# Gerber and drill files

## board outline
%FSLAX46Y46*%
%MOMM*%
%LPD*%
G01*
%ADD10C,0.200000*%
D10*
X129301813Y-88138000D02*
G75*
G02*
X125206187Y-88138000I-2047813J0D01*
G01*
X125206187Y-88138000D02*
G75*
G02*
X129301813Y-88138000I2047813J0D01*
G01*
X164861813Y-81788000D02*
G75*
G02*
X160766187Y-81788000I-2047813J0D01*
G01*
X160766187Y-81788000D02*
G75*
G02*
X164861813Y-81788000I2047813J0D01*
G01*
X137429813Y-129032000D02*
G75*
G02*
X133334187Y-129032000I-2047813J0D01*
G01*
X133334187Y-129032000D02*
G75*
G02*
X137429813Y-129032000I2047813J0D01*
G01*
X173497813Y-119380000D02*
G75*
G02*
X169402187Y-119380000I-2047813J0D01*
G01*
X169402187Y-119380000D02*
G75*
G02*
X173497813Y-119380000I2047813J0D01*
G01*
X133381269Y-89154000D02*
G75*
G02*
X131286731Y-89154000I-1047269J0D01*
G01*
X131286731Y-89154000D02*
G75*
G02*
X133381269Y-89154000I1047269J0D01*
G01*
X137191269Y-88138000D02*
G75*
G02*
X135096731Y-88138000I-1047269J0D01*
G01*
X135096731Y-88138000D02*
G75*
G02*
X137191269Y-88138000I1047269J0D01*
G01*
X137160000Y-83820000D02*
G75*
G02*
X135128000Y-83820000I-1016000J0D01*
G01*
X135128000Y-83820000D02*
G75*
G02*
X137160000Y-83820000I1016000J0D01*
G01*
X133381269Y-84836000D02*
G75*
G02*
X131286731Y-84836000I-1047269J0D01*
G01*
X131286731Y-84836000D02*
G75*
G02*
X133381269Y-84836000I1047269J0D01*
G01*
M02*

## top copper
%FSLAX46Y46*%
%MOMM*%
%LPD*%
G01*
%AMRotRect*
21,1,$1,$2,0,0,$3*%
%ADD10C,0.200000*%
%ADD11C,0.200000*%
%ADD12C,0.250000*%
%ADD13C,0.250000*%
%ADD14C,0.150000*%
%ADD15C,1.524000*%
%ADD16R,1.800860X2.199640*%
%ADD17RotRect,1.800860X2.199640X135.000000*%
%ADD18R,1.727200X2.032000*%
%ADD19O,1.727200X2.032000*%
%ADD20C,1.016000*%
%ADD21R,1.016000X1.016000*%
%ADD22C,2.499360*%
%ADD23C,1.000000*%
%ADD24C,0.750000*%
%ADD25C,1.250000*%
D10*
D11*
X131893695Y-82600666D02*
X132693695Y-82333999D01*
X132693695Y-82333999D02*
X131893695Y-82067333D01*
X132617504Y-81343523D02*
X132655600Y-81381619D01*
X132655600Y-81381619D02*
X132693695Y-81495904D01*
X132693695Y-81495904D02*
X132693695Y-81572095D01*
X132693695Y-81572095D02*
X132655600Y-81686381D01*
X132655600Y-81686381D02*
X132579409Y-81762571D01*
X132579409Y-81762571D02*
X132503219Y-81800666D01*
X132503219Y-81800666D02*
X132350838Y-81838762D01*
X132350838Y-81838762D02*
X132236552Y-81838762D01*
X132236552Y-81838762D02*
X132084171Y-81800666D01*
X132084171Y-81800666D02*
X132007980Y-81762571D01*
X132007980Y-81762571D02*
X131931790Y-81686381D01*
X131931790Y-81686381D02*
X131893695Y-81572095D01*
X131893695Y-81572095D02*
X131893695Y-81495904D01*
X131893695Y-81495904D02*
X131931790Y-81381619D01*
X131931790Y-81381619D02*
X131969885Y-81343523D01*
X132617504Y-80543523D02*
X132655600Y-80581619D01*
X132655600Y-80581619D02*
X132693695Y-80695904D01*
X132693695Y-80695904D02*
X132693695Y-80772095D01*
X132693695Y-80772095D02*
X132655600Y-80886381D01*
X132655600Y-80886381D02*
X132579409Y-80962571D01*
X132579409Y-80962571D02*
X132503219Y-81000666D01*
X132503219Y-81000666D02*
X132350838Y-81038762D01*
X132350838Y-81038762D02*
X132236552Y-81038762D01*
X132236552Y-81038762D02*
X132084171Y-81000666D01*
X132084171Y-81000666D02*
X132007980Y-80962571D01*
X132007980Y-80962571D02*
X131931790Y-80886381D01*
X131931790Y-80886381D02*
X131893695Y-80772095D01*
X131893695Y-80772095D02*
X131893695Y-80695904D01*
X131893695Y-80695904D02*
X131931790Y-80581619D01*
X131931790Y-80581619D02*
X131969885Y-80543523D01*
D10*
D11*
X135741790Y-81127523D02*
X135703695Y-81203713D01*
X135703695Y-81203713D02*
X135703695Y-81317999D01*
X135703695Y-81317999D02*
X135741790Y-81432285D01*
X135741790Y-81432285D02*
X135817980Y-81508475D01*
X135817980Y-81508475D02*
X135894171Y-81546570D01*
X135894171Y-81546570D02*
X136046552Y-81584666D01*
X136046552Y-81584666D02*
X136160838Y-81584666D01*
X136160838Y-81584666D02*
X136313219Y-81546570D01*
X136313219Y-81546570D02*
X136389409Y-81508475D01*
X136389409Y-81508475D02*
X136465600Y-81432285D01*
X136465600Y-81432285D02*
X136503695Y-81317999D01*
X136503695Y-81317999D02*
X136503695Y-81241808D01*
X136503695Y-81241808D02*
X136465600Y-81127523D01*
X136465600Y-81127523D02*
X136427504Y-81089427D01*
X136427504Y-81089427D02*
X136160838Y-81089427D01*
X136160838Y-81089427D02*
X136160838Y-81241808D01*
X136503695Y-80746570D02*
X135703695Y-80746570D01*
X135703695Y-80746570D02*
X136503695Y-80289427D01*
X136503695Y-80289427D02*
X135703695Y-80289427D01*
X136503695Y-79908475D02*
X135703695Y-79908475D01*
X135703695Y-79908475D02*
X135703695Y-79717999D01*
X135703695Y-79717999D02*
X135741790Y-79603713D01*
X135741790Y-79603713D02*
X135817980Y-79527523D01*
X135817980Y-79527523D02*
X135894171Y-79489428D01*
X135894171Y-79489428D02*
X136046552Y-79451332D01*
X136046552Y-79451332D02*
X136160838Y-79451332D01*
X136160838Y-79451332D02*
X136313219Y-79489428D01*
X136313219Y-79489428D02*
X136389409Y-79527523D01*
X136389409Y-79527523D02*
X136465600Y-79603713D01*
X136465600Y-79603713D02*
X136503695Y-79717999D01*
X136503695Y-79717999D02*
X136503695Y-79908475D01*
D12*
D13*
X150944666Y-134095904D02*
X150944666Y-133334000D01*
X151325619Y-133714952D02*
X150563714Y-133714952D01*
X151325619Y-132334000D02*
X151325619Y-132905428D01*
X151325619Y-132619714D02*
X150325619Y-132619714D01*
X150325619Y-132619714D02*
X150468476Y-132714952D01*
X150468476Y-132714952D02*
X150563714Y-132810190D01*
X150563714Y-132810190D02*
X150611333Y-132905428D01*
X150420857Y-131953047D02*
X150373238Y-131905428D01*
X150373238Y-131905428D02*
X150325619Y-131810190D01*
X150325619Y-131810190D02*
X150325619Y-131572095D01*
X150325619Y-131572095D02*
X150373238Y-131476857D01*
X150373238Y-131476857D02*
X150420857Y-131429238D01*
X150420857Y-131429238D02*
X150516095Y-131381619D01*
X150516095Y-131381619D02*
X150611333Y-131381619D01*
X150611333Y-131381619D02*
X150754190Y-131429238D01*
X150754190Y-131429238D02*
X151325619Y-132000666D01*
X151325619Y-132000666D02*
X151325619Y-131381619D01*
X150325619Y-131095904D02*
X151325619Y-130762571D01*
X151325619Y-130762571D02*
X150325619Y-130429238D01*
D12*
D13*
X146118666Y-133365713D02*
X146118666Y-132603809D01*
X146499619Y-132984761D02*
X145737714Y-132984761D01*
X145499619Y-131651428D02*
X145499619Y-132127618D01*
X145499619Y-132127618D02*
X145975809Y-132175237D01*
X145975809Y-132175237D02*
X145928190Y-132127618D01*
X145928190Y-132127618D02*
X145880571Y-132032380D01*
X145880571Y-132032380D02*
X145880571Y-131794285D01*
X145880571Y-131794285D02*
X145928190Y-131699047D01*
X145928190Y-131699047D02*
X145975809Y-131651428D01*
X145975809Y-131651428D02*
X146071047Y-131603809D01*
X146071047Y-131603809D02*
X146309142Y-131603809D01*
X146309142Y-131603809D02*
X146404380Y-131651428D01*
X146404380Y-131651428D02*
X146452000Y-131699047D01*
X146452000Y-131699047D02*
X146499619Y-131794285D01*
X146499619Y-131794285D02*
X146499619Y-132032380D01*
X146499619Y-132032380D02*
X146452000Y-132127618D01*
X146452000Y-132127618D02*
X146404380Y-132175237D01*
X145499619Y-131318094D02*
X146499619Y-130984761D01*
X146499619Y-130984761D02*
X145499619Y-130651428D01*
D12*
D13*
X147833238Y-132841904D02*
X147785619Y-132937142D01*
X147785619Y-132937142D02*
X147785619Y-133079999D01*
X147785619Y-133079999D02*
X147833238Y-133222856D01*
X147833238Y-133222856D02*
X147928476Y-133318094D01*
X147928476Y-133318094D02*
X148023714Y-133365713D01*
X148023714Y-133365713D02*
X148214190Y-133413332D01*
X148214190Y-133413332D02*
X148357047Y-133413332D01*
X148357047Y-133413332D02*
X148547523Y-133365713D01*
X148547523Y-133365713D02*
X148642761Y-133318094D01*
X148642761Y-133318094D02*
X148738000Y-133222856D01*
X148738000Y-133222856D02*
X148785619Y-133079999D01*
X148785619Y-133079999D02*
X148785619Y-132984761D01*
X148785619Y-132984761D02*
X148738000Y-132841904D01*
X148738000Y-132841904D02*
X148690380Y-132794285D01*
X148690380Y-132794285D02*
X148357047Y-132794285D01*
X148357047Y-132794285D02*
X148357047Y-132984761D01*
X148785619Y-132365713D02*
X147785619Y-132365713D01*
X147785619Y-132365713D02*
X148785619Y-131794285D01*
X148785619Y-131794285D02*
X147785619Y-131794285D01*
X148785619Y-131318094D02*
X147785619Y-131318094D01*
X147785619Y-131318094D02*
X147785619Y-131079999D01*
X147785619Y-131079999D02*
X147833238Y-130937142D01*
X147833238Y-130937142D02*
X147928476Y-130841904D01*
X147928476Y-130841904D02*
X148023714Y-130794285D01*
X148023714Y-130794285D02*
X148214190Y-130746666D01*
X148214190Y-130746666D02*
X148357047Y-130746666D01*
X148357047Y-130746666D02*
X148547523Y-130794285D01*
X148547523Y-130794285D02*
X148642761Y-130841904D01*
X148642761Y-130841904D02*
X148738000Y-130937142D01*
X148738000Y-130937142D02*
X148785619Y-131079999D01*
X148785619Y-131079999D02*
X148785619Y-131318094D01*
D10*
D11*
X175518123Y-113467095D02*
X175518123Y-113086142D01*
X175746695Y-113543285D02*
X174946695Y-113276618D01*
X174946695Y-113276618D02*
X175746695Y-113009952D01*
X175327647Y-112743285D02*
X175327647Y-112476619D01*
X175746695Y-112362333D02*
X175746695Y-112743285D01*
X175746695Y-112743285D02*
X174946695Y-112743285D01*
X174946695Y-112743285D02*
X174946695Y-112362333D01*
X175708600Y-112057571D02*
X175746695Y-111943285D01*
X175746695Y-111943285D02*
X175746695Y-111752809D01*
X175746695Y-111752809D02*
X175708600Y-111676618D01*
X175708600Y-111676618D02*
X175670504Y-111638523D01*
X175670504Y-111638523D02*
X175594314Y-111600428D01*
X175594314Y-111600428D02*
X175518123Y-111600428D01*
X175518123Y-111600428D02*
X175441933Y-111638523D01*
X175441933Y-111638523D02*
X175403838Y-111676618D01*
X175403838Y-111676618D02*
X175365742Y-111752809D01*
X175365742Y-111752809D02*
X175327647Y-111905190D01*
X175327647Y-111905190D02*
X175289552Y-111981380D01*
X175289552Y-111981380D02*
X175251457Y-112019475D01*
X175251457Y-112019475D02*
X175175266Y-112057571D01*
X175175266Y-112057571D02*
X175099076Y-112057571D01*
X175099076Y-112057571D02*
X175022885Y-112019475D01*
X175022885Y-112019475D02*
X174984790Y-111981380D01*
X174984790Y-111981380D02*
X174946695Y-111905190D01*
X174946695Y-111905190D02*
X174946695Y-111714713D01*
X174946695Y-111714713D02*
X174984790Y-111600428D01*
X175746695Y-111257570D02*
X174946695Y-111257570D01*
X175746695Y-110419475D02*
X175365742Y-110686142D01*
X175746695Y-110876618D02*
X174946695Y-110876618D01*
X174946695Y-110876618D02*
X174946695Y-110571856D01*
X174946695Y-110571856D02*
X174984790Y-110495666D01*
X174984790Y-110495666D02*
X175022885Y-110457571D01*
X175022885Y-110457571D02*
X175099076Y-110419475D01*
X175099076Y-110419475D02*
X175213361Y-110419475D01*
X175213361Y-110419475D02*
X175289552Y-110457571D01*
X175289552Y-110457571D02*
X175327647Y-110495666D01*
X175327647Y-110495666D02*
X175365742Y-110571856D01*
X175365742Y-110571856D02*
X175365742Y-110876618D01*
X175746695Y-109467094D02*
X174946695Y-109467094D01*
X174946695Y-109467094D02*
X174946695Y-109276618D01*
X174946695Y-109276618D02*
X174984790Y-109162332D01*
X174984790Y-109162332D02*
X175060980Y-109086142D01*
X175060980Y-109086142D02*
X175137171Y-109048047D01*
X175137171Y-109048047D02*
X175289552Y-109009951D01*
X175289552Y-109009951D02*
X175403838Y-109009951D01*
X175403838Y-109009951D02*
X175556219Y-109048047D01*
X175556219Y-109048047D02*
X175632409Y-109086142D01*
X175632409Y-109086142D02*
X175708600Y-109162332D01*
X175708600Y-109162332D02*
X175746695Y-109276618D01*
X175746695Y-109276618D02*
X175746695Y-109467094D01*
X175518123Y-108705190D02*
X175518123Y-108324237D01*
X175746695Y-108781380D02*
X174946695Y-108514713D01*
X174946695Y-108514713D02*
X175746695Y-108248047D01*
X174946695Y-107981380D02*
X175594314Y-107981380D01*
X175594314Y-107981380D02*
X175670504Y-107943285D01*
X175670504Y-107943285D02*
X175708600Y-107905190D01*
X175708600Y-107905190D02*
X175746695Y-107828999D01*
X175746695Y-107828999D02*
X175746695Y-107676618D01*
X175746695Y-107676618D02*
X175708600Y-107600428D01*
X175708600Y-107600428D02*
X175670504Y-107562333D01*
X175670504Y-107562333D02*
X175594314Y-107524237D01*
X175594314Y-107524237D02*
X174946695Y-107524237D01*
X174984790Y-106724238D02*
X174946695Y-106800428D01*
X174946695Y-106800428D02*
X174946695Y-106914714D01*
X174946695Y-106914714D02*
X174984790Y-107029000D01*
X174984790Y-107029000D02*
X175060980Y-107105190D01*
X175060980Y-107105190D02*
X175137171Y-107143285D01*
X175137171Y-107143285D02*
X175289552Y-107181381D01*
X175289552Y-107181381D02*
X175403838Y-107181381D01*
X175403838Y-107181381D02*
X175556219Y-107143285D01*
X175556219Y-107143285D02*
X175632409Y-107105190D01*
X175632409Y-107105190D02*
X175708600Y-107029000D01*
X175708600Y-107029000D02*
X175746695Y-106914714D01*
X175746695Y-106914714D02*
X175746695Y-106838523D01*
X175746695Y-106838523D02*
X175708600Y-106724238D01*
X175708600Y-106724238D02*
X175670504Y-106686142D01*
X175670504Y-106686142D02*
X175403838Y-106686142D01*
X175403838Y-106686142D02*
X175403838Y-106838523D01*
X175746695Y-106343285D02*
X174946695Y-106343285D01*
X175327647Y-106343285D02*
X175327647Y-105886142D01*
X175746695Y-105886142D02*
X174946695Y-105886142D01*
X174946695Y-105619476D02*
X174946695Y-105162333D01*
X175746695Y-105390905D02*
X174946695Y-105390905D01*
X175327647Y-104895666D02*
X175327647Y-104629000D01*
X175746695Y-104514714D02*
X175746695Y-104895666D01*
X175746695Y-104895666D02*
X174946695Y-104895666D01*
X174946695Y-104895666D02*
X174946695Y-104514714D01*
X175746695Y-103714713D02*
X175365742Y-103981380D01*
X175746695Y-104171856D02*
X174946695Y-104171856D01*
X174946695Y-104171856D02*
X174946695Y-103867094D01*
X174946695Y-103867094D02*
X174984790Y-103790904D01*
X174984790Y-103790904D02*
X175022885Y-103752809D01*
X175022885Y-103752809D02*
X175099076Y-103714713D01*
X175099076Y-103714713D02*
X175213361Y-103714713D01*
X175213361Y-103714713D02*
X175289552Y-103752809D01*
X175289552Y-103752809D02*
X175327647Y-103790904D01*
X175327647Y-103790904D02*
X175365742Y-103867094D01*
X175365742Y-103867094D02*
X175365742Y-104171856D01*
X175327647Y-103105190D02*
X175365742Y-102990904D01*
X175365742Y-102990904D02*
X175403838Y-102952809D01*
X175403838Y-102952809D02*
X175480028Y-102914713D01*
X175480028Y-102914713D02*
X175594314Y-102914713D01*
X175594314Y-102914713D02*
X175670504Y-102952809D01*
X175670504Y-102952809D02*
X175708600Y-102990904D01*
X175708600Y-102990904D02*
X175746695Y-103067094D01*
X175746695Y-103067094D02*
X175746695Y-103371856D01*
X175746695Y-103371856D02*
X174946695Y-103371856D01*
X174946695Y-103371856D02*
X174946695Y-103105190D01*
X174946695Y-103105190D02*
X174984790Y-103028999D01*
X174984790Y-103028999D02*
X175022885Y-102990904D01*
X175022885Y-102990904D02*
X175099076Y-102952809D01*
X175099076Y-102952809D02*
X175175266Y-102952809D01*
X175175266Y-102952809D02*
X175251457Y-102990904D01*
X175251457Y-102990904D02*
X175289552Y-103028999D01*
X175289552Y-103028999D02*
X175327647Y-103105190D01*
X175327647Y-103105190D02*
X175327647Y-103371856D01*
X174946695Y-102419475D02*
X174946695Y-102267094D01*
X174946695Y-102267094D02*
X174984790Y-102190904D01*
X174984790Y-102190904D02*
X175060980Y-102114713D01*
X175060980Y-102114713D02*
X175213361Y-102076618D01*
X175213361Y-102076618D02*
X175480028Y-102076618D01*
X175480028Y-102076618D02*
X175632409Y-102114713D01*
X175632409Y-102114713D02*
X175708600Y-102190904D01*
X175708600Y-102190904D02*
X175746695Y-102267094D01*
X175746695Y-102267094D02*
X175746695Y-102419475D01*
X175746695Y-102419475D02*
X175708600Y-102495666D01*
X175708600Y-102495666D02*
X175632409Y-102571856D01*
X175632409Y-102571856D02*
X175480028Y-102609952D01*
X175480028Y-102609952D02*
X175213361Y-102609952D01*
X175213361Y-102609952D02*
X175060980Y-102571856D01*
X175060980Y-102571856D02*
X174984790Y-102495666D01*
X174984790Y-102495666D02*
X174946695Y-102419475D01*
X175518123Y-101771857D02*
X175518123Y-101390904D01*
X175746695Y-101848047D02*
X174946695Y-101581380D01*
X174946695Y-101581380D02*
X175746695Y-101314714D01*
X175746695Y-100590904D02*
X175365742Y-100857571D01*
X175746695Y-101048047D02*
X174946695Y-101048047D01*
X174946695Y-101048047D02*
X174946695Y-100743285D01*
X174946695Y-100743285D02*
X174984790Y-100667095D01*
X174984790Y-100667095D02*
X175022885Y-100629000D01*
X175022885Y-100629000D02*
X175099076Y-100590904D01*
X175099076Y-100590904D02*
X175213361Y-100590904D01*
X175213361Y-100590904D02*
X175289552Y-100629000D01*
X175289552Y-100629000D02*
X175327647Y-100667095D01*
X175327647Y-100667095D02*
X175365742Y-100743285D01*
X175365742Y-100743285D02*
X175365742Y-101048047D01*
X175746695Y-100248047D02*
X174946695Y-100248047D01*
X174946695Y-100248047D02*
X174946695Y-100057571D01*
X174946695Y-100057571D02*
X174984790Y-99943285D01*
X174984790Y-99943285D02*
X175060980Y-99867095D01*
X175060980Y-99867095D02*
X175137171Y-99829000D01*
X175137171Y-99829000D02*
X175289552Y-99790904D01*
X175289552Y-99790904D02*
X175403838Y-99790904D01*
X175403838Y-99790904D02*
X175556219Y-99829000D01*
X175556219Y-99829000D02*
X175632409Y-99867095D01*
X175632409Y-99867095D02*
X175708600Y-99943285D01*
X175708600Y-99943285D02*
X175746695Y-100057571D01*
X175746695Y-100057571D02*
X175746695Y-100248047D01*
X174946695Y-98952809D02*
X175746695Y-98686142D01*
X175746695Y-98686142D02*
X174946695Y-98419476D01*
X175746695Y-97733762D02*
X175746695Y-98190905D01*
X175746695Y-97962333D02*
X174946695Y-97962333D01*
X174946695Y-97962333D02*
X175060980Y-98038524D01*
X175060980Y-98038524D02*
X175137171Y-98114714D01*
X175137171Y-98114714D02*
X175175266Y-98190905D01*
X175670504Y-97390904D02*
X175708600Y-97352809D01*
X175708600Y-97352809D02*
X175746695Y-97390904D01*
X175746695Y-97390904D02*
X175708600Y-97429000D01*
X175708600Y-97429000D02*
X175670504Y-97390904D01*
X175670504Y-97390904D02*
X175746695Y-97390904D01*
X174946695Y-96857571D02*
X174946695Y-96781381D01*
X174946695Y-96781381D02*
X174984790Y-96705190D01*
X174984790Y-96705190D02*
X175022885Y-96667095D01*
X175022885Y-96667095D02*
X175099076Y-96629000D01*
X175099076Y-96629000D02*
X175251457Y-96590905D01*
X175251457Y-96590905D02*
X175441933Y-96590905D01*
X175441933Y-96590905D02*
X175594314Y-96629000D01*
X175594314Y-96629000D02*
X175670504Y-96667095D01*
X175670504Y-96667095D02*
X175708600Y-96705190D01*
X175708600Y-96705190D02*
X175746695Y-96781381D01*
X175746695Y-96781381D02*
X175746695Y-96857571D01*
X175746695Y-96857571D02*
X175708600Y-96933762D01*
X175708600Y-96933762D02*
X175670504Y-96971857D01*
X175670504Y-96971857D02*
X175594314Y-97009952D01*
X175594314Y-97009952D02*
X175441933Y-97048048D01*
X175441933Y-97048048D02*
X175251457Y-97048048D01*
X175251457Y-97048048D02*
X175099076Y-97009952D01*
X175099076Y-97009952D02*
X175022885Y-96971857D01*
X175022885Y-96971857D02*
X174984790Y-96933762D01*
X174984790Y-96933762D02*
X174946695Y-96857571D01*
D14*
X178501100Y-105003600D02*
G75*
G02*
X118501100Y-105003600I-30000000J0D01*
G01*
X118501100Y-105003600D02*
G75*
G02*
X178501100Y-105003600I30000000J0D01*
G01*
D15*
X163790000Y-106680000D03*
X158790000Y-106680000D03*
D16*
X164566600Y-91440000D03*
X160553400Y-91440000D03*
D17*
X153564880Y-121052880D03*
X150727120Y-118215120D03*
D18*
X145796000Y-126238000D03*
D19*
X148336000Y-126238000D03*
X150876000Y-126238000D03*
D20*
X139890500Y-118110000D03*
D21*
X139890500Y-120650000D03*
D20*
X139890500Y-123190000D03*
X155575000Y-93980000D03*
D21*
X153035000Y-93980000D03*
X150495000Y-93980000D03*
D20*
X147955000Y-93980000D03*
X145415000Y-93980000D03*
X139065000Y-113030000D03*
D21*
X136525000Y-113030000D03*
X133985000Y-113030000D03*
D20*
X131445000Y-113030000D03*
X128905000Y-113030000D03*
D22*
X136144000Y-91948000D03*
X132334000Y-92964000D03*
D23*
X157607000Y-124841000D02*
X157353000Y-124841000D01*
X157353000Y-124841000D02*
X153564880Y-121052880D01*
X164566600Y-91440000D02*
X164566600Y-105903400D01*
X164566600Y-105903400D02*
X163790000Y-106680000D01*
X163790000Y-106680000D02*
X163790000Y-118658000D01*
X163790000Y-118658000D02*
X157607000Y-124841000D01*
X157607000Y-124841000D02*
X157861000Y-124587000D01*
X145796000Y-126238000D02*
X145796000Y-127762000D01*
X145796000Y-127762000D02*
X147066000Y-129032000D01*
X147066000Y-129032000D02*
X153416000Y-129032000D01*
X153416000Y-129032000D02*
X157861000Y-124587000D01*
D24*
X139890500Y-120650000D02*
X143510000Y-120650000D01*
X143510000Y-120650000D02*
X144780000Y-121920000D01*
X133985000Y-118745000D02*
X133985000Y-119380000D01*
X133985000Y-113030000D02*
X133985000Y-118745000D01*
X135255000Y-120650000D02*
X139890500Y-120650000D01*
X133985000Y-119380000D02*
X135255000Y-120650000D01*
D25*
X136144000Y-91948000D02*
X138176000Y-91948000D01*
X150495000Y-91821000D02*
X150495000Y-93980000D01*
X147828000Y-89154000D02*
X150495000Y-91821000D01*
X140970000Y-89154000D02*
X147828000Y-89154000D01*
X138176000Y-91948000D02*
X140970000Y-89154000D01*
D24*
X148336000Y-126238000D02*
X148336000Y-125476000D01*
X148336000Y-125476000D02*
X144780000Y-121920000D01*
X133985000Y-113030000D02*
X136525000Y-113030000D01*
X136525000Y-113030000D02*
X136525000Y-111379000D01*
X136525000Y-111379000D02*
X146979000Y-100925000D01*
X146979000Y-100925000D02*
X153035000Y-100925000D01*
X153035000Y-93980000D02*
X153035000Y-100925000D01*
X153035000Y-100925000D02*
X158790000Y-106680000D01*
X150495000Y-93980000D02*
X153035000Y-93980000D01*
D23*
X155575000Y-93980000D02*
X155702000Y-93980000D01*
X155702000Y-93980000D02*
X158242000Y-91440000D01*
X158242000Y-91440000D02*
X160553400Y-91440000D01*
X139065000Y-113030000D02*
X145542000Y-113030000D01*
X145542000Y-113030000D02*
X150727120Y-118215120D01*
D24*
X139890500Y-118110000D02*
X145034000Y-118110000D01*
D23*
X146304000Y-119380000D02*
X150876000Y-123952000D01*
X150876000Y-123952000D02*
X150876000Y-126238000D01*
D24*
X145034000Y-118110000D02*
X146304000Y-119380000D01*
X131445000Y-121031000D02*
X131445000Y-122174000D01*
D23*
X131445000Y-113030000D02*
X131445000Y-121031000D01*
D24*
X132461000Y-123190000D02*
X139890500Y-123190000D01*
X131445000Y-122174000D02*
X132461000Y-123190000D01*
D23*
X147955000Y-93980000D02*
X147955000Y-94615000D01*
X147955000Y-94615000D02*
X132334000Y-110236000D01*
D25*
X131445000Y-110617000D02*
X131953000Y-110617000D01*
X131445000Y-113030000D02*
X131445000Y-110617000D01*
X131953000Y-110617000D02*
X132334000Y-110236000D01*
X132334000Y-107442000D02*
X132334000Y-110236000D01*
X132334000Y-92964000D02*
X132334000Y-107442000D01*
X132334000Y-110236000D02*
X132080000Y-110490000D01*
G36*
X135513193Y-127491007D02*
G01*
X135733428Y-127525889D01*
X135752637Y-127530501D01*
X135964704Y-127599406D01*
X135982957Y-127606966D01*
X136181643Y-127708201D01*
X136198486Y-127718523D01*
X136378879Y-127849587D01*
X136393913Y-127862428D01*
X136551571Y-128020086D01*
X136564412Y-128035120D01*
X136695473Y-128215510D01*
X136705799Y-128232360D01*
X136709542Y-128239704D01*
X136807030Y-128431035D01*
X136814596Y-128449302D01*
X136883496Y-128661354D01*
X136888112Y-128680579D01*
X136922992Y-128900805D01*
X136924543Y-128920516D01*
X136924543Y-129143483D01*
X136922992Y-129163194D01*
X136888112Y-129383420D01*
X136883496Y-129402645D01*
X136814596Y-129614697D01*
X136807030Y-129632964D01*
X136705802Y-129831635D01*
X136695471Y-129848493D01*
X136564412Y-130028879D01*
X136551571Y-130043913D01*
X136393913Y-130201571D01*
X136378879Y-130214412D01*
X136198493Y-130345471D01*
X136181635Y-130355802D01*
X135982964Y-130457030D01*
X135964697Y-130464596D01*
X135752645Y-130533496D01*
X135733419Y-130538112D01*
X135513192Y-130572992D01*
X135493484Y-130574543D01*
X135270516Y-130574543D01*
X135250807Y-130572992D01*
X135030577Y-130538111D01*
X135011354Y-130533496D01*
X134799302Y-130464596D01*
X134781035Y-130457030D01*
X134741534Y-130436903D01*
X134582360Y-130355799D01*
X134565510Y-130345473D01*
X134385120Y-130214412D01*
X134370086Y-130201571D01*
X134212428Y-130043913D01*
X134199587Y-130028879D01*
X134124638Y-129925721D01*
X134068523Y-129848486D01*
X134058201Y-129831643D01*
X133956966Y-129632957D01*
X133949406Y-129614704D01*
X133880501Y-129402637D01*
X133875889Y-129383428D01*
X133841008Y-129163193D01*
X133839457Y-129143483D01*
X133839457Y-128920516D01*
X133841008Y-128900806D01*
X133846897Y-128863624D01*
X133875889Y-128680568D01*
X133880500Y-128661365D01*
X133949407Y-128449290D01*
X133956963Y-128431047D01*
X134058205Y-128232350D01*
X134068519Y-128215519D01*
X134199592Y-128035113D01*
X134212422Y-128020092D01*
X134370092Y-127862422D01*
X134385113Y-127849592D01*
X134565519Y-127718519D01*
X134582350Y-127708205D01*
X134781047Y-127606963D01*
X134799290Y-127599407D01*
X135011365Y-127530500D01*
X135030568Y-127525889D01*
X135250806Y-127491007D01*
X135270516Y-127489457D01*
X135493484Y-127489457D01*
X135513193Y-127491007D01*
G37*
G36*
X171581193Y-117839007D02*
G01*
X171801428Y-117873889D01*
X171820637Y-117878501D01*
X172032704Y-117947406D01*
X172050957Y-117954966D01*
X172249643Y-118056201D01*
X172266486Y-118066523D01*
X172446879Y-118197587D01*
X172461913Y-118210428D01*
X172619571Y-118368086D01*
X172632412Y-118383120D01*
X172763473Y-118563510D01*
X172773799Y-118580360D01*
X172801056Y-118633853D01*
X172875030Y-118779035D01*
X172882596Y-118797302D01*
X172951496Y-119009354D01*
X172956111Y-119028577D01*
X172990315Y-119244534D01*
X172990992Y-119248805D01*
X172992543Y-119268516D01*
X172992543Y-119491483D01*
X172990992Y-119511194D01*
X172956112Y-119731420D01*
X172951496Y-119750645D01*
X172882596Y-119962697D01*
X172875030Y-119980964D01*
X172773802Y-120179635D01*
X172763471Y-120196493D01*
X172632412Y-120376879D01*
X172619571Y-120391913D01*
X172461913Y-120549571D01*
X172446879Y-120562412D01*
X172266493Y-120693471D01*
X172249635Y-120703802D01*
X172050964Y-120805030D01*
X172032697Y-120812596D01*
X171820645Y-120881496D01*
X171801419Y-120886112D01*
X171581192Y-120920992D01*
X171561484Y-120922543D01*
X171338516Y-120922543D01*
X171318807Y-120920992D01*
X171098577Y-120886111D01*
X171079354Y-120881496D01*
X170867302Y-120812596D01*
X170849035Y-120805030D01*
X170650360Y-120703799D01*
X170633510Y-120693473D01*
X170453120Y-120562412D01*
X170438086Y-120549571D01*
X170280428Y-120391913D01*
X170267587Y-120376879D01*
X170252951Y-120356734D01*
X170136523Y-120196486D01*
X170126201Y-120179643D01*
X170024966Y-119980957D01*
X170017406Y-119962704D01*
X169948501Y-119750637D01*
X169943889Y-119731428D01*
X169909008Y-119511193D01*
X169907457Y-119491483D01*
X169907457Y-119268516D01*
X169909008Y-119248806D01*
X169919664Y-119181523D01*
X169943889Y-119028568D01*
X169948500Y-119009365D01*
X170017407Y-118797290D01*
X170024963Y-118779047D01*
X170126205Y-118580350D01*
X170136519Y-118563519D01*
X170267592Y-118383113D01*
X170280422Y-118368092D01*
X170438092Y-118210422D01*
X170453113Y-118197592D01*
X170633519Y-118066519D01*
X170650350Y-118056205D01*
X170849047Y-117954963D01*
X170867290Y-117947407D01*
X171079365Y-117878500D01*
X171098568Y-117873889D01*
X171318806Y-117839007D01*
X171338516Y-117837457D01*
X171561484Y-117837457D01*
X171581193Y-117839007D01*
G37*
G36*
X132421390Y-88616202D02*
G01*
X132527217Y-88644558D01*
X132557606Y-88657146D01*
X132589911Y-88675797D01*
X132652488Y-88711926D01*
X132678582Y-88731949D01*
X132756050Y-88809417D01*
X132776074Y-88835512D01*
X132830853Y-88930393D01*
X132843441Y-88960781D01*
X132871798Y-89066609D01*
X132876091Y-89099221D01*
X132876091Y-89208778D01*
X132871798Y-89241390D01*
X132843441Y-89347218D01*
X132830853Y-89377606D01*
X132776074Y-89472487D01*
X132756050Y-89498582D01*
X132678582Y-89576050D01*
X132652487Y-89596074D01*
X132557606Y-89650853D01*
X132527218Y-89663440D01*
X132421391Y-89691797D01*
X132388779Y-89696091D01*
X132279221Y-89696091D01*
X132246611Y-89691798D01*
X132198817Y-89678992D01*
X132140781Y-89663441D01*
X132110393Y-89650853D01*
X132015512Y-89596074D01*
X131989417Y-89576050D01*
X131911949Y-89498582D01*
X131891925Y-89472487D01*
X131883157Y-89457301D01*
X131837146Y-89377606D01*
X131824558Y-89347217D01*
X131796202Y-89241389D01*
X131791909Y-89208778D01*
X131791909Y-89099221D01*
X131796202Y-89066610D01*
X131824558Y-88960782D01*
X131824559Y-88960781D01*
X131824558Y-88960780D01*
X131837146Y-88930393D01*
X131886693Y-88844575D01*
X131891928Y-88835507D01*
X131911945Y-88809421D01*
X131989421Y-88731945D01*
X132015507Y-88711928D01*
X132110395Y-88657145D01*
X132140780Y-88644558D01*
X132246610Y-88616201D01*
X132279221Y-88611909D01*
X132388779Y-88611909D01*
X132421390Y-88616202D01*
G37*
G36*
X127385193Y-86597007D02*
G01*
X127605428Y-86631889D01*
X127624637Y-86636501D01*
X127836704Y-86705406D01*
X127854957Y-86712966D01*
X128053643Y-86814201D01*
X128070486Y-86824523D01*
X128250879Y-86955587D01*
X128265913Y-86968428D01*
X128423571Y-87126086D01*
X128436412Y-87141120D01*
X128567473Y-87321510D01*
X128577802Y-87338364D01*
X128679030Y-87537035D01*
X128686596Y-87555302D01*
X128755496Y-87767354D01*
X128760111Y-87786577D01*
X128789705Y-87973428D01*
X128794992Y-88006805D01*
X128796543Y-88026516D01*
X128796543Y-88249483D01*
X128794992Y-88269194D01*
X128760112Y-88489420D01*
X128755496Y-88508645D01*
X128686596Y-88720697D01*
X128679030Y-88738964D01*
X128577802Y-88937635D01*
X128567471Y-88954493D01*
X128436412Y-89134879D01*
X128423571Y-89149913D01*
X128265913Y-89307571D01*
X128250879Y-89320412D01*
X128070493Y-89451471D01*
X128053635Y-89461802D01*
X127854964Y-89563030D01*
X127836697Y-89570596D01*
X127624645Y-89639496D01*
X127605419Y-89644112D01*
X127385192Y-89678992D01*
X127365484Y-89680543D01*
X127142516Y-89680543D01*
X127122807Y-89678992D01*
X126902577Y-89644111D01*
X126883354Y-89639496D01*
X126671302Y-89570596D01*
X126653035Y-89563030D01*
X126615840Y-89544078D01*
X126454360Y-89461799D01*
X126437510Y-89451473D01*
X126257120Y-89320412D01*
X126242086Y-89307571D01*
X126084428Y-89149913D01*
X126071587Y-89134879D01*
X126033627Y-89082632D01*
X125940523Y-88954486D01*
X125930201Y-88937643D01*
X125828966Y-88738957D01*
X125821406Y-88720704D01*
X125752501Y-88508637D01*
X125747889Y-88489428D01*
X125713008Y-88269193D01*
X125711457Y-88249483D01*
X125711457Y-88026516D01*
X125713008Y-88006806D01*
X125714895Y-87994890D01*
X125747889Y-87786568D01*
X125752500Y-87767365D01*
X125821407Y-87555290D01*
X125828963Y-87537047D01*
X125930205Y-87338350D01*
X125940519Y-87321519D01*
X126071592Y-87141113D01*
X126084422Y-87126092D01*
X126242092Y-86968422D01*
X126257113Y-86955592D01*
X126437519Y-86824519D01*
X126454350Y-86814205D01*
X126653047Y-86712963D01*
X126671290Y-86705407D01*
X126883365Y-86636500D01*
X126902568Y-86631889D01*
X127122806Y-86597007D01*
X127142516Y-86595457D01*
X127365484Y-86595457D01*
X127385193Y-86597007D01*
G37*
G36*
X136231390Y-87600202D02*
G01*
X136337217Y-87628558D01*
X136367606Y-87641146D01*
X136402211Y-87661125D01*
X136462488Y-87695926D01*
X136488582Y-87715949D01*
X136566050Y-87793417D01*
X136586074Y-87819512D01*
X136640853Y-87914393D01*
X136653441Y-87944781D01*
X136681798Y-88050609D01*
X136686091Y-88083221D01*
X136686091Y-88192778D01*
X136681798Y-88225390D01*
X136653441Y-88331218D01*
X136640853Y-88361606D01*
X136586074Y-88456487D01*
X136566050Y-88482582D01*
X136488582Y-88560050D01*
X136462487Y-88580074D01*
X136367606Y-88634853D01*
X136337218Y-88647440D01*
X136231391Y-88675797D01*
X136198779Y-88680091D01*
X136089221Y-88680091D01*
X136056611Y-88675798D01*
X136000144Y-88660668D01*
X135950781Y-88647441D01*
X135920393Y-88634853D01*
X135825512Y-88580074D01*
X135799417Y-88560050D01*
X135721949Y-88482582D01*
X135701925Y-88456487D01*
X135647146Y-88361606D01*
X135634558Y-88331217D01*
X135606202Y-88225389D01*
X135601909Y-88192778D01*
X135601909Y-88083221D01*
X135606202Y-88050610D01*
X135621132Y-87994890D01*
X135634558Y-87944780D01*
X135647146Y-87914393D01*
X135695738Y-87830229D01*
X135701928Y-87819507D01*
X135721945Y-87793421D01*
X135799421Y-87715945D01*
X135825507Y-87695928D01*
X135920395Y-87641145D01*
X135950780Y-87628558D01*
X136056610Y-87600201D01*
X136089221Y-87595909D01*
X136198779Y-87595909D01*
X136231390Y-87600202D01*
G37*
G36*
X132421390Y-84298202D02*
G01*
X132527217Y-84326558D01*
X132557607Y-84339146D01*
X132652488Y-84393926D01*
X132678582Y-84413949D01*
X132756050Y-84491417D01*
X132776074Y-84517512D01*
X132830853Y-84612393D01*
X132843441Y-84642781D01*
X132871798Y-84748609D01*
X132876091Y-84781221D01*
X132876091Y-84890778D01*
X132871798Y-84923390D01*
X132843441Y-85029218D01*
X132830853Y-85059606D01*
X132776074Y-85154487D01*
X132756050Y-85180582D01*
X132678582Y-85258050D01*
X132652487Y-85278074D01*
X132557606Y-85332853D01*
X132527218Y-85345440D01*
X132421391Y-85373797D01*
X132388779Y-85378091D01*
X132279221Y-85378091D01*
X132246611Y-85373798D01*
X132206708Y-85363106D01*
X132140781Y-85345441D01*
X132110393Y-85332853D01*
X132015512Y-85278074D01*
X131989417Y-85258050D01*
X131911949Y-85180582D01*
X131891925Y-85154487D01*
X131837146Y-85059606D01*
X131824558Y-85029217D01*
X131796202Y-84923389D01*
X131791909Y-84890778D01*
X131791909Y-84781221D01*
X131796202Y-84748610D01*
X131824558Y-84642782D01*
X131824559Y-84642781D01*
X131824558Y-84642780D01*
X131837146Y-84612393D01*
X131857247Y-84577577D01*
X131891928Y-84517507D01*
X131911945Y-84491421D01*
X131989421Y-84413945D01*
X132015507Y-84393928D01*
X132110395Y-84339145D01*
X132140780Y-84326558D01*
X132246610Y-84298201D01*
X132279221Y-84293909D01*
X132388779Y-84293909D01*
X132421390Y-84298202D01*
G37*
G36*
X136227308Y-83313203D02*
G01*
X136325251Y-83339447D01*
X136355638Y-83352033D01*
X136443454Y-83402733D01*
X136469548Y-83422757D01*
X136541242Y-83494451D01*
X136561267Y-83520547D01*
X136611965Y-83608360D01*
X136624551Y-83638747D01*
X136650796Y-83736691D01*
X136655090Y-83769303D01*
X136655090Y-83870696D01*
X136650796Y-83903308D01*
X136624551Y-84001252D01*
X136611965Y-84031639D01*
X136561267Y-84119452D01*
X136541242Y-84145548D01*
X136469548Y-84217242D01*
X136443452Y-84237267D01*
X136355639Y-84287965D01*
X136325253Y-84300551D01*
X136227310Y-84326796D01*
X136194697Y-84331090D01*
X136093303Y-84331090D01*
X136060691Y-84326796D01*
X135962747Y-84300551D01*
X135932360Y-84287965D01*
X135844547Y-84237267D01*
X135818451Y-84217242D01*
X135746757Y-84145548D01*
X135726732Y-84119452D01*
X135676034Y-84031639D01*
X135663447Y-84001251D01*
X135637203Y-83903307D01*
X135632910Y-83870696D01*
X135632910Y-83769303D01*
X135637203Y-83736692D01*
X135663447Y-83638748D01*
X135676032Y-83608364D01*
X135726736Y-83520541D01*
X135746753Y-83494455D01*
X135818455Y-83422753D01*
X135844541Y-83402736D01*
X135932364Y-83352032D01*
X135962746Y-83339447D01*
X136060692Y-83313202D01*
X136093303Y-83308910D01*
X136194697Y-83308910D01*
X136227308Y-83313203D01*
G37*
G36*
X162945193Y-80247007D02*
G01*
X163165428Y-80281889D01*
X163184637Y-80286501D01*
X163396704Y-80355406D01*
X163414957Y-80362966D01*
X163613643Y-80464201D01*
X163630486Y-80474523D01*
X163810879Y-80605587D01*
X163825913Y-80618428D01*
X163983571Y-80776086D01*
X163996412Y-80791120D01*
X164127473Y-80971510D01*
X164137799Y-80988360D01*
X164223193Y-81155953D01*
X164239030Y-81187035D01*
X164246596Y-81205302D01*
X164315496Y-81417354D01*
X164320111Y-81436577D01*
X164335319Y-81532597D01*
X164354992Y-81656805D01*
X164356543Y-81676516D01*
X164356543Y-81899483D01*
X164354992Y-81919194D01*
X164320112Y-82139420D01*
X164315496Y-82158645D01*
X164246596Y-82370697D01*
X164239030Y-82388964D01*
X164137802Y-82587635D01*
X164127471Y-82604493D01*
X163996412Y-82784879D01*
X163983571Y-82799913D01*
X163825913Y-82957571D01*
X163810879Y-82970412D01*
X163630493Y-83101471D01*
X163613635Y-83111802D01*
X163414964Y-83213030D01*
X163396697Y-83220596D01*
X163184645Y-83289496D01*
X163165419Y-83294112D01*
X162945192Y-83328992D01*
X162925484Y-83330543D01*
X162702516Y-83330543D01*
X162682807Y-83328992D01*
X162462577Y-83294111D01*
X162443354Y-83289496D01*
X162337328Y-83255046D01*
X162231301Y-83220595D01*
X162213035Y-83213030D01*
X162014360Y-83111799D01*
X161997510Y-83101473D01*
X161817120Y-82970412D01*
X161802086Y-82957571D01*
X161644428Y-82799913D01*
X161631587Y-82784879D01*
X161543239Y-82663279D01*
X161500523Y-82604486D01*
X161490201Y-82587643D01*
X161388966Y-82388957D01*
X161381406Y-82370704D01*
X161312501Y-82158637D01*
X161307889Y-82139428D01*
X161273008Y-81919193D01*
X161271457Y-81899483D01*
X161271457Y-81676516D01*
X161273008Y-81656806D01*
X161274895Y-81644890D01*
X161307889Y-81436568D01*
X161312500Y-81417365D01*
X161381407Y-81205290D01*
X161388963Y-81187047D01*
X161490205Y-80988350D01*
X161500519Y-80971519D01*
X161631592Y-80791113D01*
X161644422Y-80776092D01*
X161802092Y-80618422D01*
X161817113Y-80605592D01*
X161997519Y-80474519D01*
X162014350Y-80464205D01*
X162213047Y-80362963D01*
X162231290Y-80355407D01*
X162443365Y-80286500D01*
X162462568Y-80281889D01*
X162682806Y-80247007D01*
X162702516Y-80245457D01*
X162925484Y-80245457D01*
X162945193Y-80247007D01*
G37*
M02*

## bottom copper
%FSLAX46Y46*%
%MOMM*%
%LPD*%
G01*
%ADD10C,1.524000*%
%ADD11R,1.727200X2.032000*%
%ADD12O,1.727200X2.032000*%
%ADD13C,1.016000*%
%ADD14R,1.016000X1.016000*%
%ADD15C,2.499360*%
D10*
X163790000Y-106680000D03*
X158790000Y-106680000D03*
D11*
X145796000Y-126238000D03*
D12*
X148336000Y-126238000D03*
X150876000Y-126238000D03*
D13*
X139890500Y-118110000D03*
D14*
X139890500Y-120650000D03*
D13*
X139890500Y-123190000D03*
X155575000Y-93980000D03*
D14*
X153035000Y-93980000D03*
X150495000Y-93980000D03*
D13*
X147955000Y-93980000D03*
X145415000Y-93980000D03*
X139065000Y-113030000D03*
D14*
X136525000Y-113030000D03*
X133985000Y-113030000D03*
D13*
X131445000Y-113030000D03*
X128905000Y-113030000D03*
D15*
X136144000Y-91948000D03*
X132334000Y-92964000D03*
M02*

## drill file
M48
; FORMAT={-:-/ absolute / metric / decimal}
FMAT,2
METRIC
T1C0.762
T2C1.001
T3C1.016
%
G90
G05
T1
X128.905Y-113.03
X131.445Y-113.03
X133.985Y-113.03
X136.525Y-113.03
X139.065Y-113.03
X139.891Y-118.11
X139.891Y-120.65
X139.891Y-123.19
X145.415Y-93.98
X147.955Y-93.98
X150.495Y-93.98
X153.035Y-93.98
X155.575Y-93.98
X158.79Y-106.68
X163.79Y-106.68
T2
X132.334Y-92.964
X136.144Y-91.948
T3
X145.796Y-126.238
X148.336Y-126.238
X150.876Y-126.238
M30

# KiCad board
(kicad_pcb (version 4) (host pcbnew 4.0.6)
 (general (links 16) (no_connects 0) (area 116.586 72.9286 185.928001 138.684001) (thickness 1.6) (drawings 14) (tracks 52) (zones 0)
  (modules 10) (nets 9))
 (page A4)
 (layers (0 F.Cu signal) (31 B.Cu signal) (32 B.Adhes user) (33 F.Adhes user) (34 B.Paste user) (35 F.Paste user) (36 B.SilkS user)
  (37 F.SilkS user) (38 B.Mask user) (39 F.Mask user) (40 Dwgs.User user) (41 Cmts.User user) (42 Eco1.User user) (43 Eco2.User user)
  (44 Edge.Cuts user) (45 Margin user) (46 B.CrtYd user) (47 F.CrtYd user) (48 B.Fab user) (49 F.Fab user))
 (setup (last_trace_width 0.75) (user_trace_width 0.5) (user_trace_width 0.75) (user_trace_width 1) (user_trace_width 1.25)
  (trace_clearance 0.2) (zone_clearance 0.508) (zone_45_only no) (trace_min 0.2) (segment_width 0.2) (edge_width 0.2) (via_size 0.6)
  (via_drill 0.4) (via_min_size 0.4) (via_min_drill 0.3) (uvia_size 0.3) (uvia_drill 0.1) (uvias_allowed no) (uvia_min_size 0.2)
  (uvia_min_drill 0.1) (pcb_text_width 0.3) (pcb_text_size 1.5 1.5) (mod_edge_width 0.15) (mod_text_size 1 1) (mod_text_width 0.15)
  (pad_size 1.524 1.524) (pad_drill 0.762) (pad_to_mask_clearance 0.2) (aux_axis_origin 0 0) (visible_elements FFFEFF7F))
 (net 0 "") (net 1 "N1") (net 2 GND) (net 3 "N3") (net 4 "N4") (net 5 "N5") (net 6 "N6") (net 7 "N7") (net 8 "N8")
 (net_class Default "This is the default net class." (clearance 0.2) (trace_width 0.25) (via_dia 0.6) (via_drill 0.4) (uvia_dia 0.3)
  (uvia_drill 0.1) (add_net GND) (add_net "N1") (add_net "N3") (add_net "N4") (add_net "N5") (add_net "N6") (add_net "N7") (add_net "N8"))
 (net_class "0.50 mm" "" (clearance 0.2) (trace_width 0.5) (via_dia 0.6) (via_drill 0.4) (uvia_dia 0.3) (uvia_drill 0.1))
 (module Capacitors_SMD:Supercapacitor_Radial (layer F.Cu) (at 161.29 106.68 180)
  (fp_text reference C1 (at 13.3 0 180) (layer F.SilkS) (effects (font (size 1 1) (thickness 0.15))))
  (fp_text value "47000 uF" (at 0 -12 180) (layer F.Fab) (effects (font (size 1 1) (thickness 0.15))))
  (pad 1 thru_hole circle (at -2.5 0 180) (size 1.524 1.524) (drill 0.762) (layers *.Cu *.Mask) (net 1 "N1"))
  (pad 2 thru_hole circle (at 2.5 0 180) (size 1.524 1.524) (drill 0.762) (layers *.Cu *.Mask) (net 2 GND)))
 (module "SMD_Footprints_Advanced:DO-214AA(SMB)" (layer F.Cu) (at 162.56 91.44 180)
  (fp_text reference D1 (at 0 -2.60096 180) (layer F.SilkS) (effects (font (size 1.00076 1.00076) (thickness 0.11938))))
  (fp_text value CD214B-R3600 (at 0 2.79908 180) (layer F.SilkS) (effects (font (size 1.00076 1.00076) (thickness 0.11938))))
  (pad 1 smd rect (at -2.0066 0 180) (size 1.80086 2.19964) (layers F.Cu F.Paste F.Mask) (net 1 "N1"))
  (pad 2 smd rect (at 2.0066 0 180) (size 1.80086 2.19964) (layers F.Cu F.Paste F.Mask) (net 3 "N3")))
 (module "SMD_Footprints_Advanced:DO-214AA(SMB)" (layer F.Cu) (at 152.146 119.634 135)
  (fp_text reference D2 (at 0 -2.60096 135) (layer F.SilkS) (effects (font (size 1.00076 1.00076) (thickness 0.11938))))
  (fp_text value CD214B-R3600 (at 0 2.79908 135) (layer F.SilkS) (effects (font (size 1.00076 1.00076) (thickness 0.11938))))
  (pad 1 smd rect (at -2.0066 0 135) (size 1.80086 2.19964) (layers F.Cu F.Paste F.Mask) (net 1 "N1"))
  (pad 2 smd rect (at 2.0066 0 135) (size 1.80086 2.19964) (layers F.Cu F.Paste F.Mask) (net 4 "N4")))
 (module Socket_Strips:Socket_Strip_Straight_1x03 (layer F.Cu) (at 145.796 126.238)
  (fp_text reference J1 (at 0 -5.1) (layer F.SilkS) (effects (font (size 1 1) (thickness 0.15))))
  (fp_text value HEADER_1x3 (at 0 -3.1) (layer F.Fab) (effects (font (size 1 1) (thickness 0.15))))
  (pad 1 thru_hole rect (at 0 0) (size 1.7272 2.032) (drill 1.016) (layers *.Cu *.Mask) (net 1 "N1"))
  (pad 2 thru_hole oval (at 2.54 0) (size 1.7272 2.032) (drill 1.016) (layers *.Cu *.Mask) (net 2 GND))
  (pad 3 thru_hole oval (at 5.08 0) (size 1.7272 2.032) (drill 1.016) (layers *.Cu *.Mask) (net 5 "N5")))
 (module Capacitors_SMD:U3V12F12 (layer F.Cu) (at 134.62 120.65 90)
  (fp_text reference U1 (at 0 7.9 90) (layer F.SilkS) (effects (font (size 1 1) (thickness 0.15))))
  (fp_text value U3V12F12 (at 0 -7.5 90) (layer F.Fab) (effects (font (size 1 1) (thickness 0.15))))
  (pad 1 thru_hole circle (at 2.54 5.2705 90) (size 1.016 1.016) (drill 0.762) (layers *.Cu *.Mask) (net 5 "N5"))
  (pad 2 thru_hole rect (at 0 5.2705 90) (size 1.016 1.016) (drill 0.762) (layers *.Cu *.Mask) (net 2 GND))
  (pad 3 thru_hole circle (at -2.54 5.2705 90) (size 1.016 1.016) (drill 0.762) (layers *.Cu *.Mask) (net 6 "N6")))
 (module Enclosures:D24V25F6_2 (layer F.Cu) (at 148.59 86.36)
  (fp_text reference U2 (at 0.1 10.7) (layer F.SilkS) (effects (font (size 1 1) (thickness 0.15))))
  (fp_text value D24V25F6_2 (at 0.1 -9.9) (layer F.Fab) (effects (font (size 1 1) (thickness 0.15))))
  (pad 1 thru_hole circle (at 6.985 7.62) (size 1.016 1.016) (drill 0.762) (layers *.Cu *.Mask) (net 3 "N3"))
  (pad 2 thru_hole rect (at 4.445 7.62) (size 1.016 1.016) (drill 0.762) (layers *.Cu *.Mask) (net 2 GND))
  (pad 3 thru_hole rect (at 1.905 7.62) (size 1.016 1.016) (drill 0.762) (layers *.Cu *.Mask) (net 2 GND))
  (pad 4 thru_hole circle (at -0.635 7.62) (size 1.016 1.016) (drill 0.762) (layers *.Cu *.Mask) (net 6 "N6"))
  (pad 5 thru_hole circle (at -3.175 7.62) (size 1.016 1.016) (drill 0.762) (layers *.Cu *.Mask) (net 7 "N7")))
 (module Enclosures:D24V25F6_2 (layer F.Cu) (at 132.08 105.41)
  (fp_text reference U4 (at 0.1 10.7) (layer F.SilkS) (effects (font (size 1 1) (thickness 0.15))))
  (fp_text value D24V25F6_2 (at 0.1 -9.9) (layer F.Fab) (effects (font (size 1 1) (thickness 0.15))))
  (pad 1 thru_hole circle (at 6.985 7.62) (size 1.016 1.016) (drill 0.762) (layers *.Cu *.Mask) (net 4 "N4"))
  (pad 2 thru_hole rect (at 4.445 7.62) (size 1.016 1.016) (drill 0.762) (layers *.Cu *.Mask) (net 2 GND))
  (pad 3 thru_hole rect (at 1.905 7.62) (size 1.016 1.016) (drill 0.762) (layers *.Cu *.Mask) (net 2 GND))
  (pad 4 thru_hole circle (at -0.635 7.62) (size 1.016 1.016) (drill 0.762) (layers *.Cu *.Mask) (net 6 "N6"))
  (pad 5 thru_hole circle (at -3.175 7.62) (size 1.016 1.016) (drill 0.762) (layers *.Cu *.Mask) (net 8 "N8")))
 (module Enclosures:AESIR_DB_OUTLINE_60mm (layer F.Cu) (at 148.5011 105.0036)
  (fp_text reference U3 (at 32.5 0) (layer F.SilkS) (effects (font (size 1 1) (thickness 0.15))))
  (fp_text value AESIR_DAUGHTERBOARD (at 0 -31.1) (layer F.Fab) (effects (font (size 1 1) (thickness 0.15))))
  (fp_circle (center 0 0) (end 30 0) (layer F.Cu) (width 0.15)))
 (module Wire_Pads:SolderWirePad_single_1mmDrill (layer F.Cu) (at 136.144 91.948)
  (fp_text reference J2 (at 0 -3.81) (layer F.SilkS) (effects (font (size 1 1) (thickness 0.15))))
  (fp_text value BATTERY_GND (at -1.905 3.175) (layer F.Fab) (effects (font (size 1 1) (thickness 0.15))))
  (pad 1 thru_hole circle (at 0 0) (size 2.49936 2.49936) (drill 1.00076) (layers *.Cu *.Mask) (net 2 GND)))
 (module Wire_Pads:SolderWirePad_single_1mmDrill (layer F.Cu) (at 132.334 92.964)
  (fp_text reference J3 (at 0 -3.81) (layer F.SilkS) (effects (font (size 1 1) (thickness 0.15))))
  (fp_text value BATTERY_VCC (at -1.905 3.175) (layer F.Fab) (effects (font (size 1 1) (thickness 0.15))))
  (pad 1 thru_hole circle (at 0 0) (size 2.49936 2.49936) (drill 1.00076) (layers *.Cu *.Mask) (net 6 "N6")))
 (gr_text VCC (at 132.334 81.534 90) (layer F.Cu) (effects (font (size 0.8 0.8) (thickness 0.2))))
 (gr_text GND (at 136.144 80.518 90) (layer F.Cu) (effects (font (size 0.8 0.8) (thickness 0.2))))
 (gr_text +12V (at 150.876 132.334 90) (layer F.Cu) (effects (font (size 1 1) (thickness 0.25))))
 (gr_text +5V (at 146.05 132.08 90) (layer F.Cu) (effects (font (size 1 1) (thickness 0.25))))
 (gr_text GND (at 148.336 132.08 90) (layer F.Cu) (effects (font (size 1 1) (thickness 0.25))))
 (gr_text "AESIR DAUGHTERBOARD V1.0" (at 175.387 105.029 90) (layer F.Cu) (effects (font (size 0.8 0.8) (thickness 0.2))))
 (gr_circle (center 127.254 88.138) (end 127.508 86.106) (layer Edge.Cuts) (width 0.2))
 (gr_circle (center 162.814 81.788) (end 163.068 79.756) (layer Edge.Cuts) (width 0.2))
 (gr_circle (center 135.382 129.032) (end 135.636 127) (layer Edge.Cuts) (width 0.2))
 (gr_circle (center 171.45 119.38) (end 171.704 117.348) (layer Edge.Cuts) (width 0.2))
 (gr_circle (center 132.334 89.154) (end 132.588 88.138) (layer Edge.Cuts) (width 0.2))
 (gr_circle (center 136.144 88.138) (end 136.398 87.122) (layer Edge.Cuts) (width 0.2))
 (gr_circle (center 136.144 83.82) (end 136.144 82.804) (layer Edge.Cuts) (width 0.2))
 (gr_circle (center 132.334 84.836) (end 132.588 83.82) (layer Edge.Cuts) (width 0.2))
 (segment (start 157.607 124.841) (end 157.353 124.841) (width 1) (layer F.Cu) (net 1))
 (segment (start 157.353 124.841) (end 153.56488 121.05288) (width 1) (layer F.Cu) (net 1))
 (segment (start 164.5666 91.44) (end 164.5666 105.9034) (width 1) (layer F.Cu) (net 1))
 (segment (start 164.5666 105.9034) (end 163.79 106.68) (width 1) (layer F.Cu) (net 1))
 (segment (start 163.79 106.68) (end 163.79 118.658) (width 1) (layer F.Cu) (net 1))
 (segment (start 163.79 118.658) (end 157.607 124.841) (width 1) (layer F.Cu) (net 1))
 (segment (start 157.607 124.841) (end 157.861 124.587) (width 1) (layer F.Cu) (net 1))
 (segment (start 145.796 126.238) (end 145.796 127.762) (width 1) (layer F.Cu) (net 1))
 (segment (start 145.796 127.762) (end 147.066 129.032) (width 1) (layer F.Cu) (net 1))
 (segment (start 147.066 129.032) (end 153.416 129.032) (width 1) (layer F.Cu) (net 1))
 (segment (start 153.416 129.032) (end 157.861 124.587) (width 1) (layer F.Cu) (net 1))
 (segment (start 139.8905 120.65) (end 143.51 120.65) (width 0.75) (layer F.Cu) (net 2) (status 400000))
 (segment (start 143.51 120.65) (end 144.78 121.92) (width 0.75) (layer F.Cu) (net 2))
 (segment (start 133.985 118.745) (end 133.985 119.38) (width 0.75) (layer F.Cu) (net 2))
 (segment (start 133.985 113.03) (end 133.985 118.745) (width 0.75) (layer F.Cu) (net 2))
 (segment (start 135.255 120.65) (end 139.8905 120.65) (width 0.75) (layer F.Cu) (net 2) (status 800000))
 (segment (start 133.985 119.38) (end 135.255 120.65) (width 0.75) (layer F.Cu) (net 2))
 (segment (start 136.144 91.948) (end 138.176 91.948) (width 1.25) (layer F.Cu) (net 2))
 (segment (start 150.495 91.821) (end 150.495 93.98) (width 1.25) (layer F.Cu) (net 2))
 (segment (start 147.828 89.154) (end 150.495 91.821) (width 1.25) (layer F.Cu) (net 2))
 (segment (start 140.97 89.154) (end 147.828 89.154) (width 1.25) (layer F.Cu) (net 2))
 (segment (start 138.176 91.948) (end 140.97 89.154) (width 1.25) (layer F.Cu) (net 2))
 (segment (start 148.336 126.238) (end 148.336 125.476) (width 0.75) (layer F.Cu) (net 2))
 (segment (start 148.336 125.476) (end 144.78 121.92) (width 0.75) (layer F.Cu) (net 2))
 (segment (start 133.985 113.03) (end 136.525 113.03) (width 0.75) (layer F.Cu) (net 2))
 (segment (start 136.525 113.03) (end 136.525 111.379) (width 0.75) (layer F.Cu) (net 2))
 (segment (start 136.525 111.379) (end 146.979 100.925) (width 0.75) (layer F.Cu) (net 2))
 (segment (start 146.979 100.925) (end 153.035 100.925) (width 0.75) (layer F.Cu) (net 2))
 (segment (start 153.035 93.98) (end 153.035 100.925) (width 0.75) (layer F.Cu) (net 2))
 (segment (start 153.035 100.925) (end 158.79 106.68) (width 0.75) (layer F.Cu) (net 2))
 (segment (start 150.495 93.98) (end 153.035 93.98) (width 0.75) (layer F.Cu) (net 2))
 (segment (start 155.575 93.98) (end 155.702 93.98) (width 1) (layer F.Cu) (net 3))
 (segment (start 155.702 93.98) (end 158.242 91.44) (width 1) (layer F.Cu) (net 3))
 (segment (start 158.242 91.44) (end 160.5534 91.44) (width 1) (layer F.Cu) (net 3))
 (segment (start 139.065 113.03) (end 145.542 113.03) (width 1) (layer F.Cu) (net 4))
 (segment (start 145.542 113.03) (end 150.72712 118.21512) (width 1) (layer F.Cu) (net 4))
 (segment (start 139.8905 118.11) (end 145.034 118.11) (width 0.75) (layer F.Cu) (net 5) (status 400000))
 (segment (start 146.304 119.38) (end 150.876 123.952) (width 1) (layer F.Cu) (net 5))
 (segment (start 150.876 123.952) (end 150.876 126.238) (width 1) (layer F.Cu) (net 5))
 (segment (start 145.034 118.11) (end 146.304 119.38) (width 0.75) (layer F.Cu) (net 5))
 (segment (start 131.445 121.031) (end 131.445 122.174) (width 0.75) (layer F.Cu) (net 6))
 (segment (start 131.445 113.03) (end 131.445 121.031) (width 1) (layer F.Cu) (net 6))
 (segment (start 132.461 123.19) (end 139.8905 123.19) (width 0.75) (layer F.Cu) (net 6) (status 800000))
 (segment (start 131.445 122.174) (end 132.461 123.19) (width 0.75) (layer F.Cu) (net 6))
 (segment (start 147.955 93.98) (end 147.955 94.615) (width 1) (layer F.Cu) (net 6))
 (segment (start 147.955 94.615) (end 132.334 110.236) (width 1) (layer F.Cu) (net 6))
 (segment (start 131.445 110.617) (end 131.953 110.617) (width 1.25) (layer F.Cu) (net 6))
 (segment (start 131.445 113.03) (end 131.445 110.617) (width 1.25) (layer F.Cu) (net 6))
 (segment (start 131.953 110.617) (end 132.334 110.236) (width 1.25) (layer F.Cu) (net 6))
 (segment (start 132.334 107.442) (end 132.334 110.236) (width 1.25) (layer F.Cu) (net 6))
 (segment (start 132.334 92.964) (end 132.334 107.442) (width 1.25) (layer F.Cu) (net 6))
 (segment (start 132.334 110.236) (end 132.08 110.49) (width 1.25) (layer F.Cu) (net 6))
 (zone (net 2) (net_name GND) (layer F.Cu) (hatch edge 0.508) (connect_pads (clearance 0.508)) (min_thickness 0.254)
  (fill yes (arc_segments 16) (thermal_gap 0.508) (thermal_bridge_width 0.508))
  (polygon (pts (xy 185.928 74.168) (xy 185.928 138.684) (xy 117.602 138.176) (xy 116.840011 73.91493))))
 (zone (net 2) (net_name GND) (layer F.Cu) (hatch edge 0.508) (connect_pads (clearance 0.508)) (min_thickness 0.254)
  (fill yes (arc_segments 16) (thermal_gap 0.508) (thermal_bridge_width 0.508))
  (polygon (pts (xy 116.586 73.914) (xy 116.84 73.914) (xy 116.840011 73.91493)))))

